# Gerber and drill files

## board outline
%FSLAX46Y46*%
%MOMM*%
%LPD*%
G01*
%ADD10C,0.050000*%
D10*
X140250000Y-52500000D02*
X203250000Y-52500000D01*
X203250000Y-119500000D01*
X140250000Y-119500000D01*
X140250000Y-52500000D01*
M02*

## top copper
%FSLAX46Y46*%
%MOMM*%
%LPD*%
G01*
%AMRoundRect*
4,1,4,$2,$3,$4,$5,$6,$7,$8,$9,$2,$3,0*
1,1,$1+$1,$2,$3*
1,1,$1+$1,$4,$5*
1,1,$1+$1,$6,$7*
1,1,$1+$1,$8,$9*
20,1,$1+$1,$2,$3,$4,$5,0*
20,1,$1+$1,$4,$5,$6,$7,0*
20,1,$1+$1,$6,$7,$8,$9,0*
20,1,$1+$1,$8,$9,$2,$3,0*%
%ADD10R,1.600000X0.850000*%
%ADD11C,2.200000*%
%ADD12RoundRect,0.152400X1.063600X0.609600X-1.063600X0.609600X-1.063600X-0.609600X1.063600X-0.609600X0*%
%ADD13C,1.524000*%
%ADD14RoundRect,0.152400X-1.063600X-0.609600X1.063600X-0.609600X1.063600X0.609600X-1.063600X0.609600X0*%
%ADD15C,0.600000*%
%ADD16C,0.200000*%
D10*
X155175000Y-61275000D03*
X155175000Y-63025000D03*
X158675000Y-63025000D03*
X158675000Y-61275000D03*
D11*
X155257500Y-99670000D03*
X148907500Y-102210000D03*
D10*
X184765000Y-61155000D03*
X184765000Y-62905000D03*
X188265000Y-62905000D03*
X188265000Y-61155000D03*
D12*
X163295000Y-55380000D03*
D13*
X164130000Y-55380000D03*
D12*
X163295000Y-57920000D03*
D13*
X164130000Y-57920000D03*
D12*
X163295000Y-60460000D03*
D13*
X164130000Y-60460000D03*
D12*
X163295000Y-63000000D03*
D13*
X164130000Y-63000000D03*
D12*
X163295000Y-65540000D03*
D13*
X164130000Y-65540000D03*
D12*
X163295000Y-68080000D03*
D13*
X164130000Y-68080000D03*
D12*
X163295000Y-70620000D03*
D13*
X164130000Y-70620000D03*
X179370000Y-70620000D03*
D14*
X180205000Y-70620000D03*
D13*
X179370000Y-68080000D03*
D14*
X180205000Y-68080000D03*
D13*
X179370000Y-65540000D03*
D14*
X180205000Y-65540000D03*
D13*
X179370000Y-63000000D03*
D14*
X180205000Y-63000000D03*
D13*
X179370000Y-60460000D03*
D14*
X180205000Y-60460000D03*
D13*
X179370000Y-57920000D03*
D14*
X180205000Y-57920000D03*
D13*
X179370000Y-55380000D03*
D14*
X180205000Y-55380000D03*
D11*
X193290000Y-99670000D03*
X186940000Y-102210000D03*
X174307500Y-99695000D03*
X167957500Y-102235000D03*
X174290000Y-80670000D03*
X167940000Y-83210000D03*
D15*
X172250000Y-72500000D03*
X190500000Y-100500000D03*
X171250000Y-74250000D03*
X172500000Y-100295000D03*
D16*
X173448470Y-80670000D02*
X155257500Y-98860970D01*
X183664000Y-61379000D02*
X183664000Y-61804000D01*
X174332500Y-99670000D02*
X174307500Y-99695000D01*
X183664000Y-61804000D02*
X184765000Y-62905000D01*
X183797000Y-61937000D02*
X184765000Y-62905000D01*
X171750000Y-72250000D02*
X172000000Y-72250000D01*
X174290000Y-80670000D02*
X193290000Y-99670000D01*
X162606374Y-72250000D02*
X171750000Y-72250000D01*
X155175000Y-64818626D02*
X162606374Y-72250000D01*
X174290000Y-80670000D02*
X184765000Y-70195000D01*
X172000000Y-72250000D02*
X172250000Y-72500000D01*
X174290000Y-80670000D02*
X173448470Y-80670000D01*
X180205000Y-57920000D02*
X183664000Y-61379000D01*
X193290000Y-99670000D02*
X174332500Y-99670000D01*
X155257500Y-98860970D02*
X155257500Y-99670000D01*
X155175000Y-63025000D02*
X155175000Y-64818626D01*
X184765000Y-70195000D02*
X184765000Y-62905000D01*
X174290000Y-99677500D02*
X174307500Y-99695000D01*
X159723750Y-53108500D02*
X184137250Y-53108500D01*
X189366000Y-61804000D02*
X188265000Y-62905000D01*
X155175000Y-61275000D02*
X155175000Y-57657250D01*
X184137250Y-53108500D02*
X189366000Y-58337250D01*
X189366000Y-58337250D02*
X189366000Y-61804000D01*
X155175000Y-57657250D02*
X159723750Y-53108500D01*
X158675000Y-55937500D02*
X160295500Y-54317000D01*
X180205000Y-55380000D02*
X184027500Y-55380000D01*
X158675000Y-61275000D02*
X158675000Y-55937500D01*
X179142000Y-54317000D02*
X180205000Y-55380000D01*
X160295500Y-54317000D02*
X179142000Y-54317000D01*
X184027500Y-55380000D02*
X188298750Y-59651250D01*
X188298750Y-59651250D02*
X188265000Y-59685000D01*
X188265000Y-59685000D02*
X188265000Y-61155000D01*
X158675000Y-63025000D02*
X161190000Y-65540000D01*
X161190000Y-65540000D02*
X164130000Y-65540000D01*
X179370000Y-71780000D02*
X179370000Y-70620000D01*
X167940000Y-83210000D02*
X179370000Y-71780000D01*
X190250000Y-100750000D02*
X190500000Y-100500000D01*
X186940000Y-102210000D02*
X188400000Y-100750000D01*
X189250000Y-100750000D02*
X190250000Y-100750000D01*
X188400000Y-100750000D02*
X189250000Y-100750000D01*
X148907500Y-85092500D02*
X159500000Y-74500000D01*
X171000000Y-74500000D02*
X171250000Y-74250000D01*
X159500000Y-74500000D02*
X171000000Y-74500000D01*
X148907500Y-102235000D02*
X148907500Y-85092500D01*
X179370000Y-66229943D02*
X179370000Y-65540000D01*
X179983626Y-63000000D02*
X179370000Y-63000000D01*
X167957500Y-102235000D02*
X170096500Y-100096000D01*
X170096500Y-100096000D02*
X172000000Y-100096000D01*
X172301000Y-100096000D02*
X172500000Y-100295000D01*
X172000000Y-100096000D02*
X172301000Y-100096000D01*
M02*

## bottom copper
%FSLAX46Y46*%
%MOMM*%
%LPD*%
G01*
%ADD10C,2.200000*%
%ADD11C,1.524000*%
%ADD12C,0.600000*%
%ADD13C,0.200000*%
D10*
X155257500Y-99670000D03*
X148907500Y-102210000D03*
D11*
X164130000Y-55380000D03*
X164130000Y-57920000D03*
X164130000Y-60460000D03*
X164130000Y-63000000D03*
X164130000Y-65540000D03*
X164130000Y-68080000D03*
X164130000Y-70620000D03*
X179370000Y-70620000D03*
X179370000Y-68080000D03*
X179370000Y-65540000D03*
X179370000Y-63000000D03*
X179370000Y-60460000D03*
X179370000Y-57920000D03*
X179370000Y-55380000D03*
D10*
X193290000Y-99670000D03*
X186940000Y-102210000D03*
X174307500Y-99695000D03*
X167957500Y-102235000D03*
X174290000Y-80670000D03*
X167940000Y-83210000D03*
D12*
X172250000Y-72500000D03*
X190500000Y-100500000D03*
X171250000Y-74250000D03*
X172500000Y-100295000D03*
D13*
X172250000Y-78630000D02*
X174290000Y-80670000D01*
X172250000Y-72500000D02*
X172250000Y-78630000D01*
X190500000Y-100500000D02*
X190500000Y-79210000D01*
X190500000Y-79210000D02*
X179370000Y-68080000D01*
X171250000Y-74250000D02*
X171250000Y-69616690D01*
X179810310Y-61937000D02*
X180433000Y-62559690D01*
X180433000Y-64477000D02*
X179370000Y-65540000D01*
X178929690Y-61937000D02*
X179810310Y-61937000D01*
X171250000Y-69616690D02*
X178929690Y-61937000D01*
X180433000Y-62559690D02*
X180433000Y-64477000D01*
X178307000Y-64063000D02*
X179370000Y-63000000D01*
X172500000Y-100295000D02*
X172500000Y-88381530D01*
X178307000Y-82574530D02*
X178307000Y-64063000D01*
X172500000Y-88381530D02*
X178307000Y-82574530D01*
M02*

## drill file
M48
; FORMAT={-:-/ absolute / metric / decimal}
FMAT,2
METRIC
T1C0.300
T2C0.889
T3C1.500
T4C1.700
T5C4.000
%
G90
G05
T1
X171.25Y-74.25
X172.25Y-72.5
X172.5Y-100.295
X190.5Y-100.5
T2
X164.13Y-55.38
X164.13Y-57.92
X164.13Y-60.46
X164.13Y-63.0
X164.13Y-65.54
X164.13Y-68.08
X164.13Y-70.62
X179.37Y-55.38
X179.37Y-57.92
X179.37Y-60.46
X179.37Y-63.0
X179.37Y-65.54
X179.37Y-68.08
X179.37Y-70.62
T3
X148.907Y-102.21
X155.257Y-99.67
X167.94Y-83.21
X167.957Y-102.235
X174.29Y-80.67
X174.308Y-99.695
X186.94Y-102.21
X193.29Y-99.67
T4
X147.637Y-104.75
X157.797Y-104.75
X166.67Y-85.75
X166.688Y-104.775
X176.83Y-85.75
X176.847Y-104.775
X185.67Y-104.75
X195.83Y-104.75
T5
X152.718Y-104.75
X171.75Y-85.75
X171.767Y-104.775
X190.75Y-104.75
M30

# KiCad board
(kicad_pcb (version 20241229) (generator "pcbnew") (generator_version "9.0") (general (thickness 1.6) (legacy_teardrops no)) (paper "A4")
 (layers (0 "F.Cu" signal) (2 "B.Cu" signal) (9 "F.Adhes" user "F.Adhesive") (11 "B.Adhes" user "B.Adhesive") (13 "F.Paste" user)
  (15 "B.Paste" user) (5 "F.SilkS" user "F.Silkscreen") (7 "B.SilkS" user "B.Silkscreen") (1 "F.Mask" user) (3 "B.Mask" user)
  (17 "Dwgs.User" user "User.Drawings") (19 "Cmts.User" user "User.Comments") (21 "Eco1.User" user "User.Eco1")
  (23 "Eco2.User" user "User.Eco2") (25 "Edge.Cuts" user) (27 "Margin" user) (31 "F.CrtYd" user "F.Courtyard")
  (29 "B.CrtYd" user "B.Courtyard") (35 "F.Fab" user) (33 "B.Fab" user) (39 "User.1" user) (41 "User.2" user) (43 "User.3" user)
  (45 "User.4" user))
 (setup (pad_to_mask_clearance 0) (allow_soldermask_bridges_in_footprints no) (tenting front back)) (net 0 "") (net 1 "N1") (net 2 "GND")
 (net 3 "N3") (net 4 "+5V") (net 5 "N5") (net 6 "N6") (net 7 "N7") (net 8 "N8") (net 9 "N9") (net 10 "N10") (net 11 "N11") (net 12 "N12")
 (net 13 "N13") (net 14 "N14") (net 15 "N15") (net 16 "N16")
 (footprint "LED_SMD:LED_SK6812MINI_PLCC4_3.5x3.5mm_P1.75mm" (layer "F.Cu") (at 156.925 62.15)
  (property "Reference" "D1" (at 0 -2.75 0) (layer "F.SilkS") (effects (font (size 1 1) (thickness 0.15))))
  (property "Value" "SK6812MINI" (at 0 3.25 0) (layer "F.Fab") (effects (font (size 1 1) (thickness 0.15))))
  (pad "1" smd rect (at -1.75 -0.875) (size 1.6 0.85) (layers "F.Cu" "F.Mask" "F.Paste") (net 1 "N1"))
  (pad "2" smd rect (at -1.75 0.875) (size 1.6 0.85) (layers "F.Cu" "F.Mask" "F.Paste") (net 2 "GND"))
  (pad "3" smd rect (at 1.75 0.875) (size 1.6 0.85) (layers "F.Cu" "F.Mask" "F.Paste") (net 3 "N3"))
  (pad "4" smd rect (at 1.75 -0.875) (size 1.6 0.85) (layers "F.Cu" "F.Mask" "F.Paste") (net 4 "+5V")))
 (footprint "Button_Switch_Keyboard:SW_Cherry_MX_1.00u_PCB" (layer "F.Cu") (at 155.2575 99.67)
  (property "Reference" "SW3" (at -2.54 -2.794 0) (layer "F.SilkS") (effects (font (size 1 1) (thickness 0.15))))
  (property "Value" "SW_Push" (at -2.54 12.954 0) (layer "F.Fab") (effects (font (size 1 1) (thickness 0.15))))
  (pad "" np_thru_hole circle (at -7.62 5.08) (size 1.7 1.7) (drill 1.7) (layers "*.Cu" "*.Mask"))
  (pad "" np_thru_hole circle (at -2.54 5.08) (size 4 4) (drill 4) (layers "*.Cu" "*.Mask"))
  (pad "" np_thru_hole circle (at 2.54 5.08) (size 1.7 1.7) (drill 1.7) (layers "*.Cu" "*.Mask"))
  (pad "1" thru_hole circle (at 0 0) (size 2.2 2.2) (drill 1.5) (layers "*.Cu" "*.Mask") (remove_unused_layers no) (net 2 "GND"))
  (pad "2" thru_hole circle (at -6.35 2.54) (size 2.2 2.2) (drill 1.5) (layers "*.Cu" "*.Mask") (remove_unused_layers no) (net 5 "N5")))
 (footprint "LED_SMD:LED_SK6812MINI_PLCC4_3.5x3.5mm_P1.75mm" (layer "F.Cu") (at 186.515 62.03)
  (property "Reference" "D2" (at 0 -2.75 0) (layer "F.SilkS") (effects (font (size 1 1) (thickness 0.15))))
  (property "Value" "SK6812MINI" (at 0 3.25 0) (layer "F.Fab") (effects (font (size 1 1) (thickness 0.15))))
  (pad "1" smd rect (at -1.75 -0.875) (size 1.6 0.85) (layers "F.Cu" "F.Mask" "F.Paste") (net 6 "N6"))
  (pad "2" smd rect (at -1.75 0.875) (size 1.6 0.85) (layers "F.Cu" "F.Mask" "F.Paste") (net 2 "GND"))
  (pad "3" smd rect (at 1.75 0.875) (size 1.6 0.85) (layers "F.Cu" "F.Mask" "F.Paste") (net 1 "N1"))
  (pad "4" smd rect (at 1.75 -0.875) (size 1.6 0.85) (layers "F.Cu" "F.Mask" "F.Paste") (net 4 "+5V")))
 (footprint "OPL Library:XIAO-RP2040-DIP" (layer "F.Cu") (at 171.75 63)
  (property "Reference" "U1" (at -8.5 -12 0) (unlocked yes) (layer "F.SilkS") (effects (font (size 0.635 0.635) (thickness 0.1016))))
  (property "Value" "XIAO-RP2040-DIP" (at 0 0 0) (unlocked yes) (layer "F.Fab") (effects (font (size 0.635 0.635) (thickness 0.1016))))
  (pad "1" smd roundrect (at -8.455 -7.62 180) (size 2.432 1.524) (layers "F.Cu" "F.Mask") (roundrect_rratio 0.1) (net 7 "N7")
   (thermal_bridge_angle 45))
  (pad "1" thru_hole circle (at -7.62 -7.62 180) (size 1.524 1.524) (drill 0.889) (layers "*.Cu" "*.Mask") (remove_unused_layers no)
   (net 7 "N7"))
  (pad "2" smd roundrect (at -8.455 -5.08 180) (size 2.432 1.524) (layers "F.Cu" "F.Mask") (roundrect_rratio 0.1) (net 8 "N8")
   (thermal_bridge_angle 45))
  (pad "2" thru_hole circle (at -7.62 -5.08 180) (size 1.524 1.524) (drill 0.889) (layers "*.Cu" "*.Mask") (remove_unused_layers no)
   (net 8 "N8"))
  (pad "3" smd roundrect (at -8.455 -2.54 180) (size 2.432 1.524) (layers "F.Cu" "F.Mask") (roundrect_rratio 0.1) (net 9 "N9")
   (thermal_bridge_angle 45))
  (pad "3" thru_hole circle (at -7.62 -2.54 180) (size 1.524 1.524) (drill 0.889) (layers "*.Cu" "*.Mask") (remove_unused_layers no)
   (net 9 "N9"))
  (pad "4" smd roundrect (at -8.455 0 180) (size 2.432 1.524) (layers "F.Cu" "F.Mask") (roundrect_rratio 0.1) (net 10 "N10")
   (thermal_bridge_angle 45))
  (pad "4" thru_hole circle (at -7.62 0 180) (size 1.524 1.524) (drill 0.889) (layers "*.Cu" "*.Mask") (remove_unused_layers no)
   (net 10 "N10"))
  (pad "5" smd roundrect (at -8.455 2.54 180) (size 2.432 1.524) (layers "F.Cu" "F.Mask") (roundrect_rratio 0.1) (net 3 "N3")
   (thermal_bridge_angle 45))
  (pad "5" thru_hole circle (at -7.62 2.54 180) (size 1.524 1.524) (drill 0.889) (layers "*.Cu" "*.Mask") (remove_unused_layers no)
   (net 3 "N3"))
  (pad "6" smd roundrect (at -8.455 5.08 180) (size 2.432 1.524) (layers "F.Cu" "F.Mask") (roundrect_rratio 0.1) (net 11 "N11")
   (thermal_bridge_angle 45))
  (pad "6" thru_hole circle (at -7.62 5.08 180) (size 1.524 1.524) (drill 0.889) (layers "*.Cu" "*.Mask") (remove_unused_layers no)
   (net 11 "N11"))
  (pad "7" smd roundrect (at -8.455 7.62 180) (size 2.432 1.524) (layers "F.Cu" "F.Mask") (roundrect_rratio 0.1) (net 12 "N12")
   (thermal_bridge_angle 45))
  (pad "7" thru_hole circle (at -7.62 7.62 180) (size 1.524 1.524) (drill 0.889) (layers "*.Cu" "*.Mask") (remove_unused_layers no)
   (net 12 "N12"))
  (pad "8" thru_hole circle (at 7.62 7.62) (size 1.524 1.524) (drill 0.889) (layers "*.Cu" "*.Mask") (remove_unused_layers no)
   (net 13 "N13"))
  (pad "8" smd roundrect (at 8.455 7.62) (size 2.432 1.524) (layers "F.Cu" "F.Mask") (roundrect_rratio 0.1) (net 13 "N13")
   (thermal_bridge_angle 45))
  (pad "9" thru_hole circle (at 7.62 5.08) (size 1.524 1.524) (drill 0.889) (layers "*.Cu" "*.Mask") (remove_unused_layers no)
   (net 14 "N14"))
  (pad "9" smd roundrect (at 8.455 5.08) (size 2.432 1.524) (layers "F.Cu" "F.Mask") (roundrect_rratio 0.1) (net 14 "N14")
   (thermal_bridge_angle 45))
  (pad "10" thru_hole circle (at 7.62 2.54) (size 1.524 1.524) (drill 0.889) (layers "*.Cu" "*.Mask") (remove_unused_layers no) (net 5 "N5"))
  (pad "10" smd roundrect (at 8.455 2.54) (size 2.432 1.524) (layers "F.Cu" "F.Mask") (roundrect_rratio 0.1) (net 5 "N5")
   (thermal_bridge_angle 45))
  (pad "11" thru_hole circle (at 7.62 0) (size 1.524 1.524) (drill 0.889) (layers "*.Cu" "*.Mask") (remove_unused_layers no) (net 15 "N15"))
  (pad "11" smd roundrect (at 8.455 0) (size 2.432 1.524) (layers "F.Cu" "F.Mask") (roundrect_rratio 0.1) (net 15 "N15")
   (thermal_bridge_angle 45))
  (pad "12" thru_hole circle (at 7.62 -2.54) (size 1.524 1.524) (drill 0.889) (layers "*.Cu" "*.Mask") (remove_unused_layers no)
   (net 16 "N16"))
  (pad "12" smd roundrect (at 8.455 -2.54) (size 2.432 1.524) (layers "F.Cu" "F.Mask") (roundrect_rratio 0.1) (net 16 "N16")
   (thermal_bridge_angle 45))
  (pad "13" thru_hole circle (at 7.62 -5.08) (size 1.524 1.524) (drill 0.889) (layers "*.Cu" "*.Mask") (remove_unused_layers no)
   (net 2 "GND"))
  (pad "13" smd roundrect (at 8.455 -5.08) (size 2.432 1.524) (layers "F.Cu" "F.Mask") (roundrect_rratio 0.1) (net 2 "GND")
   (thermal_bridge_angle 45))
  (pad "14" thru_hole circle (at 7.62 -7.62) (size 1.524 1.524) (drill 0.889) (layers "*.Cu" "*.Mask") (remove_unused_layers no)
   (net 4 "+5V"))
  (pad "14" smd roundrect (at 8.455 -7.62) (size 2.432 1.524) (layers "F.Cu" "F.Mask") (roundrect_rratio 0.1) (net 4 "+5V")
   (thermal_bridge_angle 45)))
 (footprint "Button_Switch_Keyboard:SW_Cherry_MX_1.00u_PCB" (layer "F.Cu") (at 193.29 99.67)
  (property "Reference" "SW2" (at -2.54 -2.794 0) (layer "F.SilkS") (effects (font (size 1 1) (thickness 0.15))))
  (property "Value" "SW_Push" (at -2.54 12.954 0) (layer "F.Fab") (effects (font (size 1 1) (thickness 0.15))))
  (pad "" np_thru_hole circle (at -7.62 5.08) (size 1.7 1.7) (drill 1.7) (layers "*.Cu" "*.Mask"))
  (pad "" np_thru_hole circle (at -2.54 5.08) (size 4 4) (drill 4) (layers "*.Cu" "*.Mask"))
  (pad "" np_thru_hole circle (at 2.54 5.08) (size 1.7 1.7) (drill 1.7) (layers "*.Cu" "*.Mask"))
  (pad "1" thru_hole circle (at 0 0) (size 2.2 2.2) (drill 1.5) (layers "*.Cu" "*.Mask") (remove_unused_layers no) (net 2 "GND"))
  (pad "2" thru_hole circle (at -6.35 2.54) (size 2.2 2.2) (drill 1.5) (layers "*.Cu" "*.Mask") (remove_unused_layers no) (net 14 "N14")))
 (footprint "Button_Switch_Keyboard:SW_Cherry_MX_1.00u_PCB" (layer "F.Cu") (at 174.3075 99.695)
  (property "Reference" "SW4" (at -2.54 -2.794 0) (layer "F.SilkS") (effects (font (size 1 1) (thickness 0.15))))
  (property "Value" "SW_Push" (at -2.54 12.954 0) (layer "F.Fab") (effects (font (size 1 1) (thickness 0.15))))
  (pad "" np_thru_hole circle (at -7.62 5.08) (size 1.7 1.7) (drill 1.7) (layers "*.Cu" "*.Mask"))
  (pad "" np_thru_hole circle (at -2.54 5.08) (size 4 4) (drill 4) (layers "*.Cu" "*.Mask"))
  (pad "" np_thru_hole circle (at 2.54 5.08) (size 1.7 1.7) (drill 1.7) (layers "*.Cu" "*.Mask"))
  (pad "1" thru_hole circle (at 0 0) (size 2.2 2.2) (drill 1.5) (layers "*.Cu" "*.Mask") (remove_unused_layers no) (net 2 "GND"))
  (pad "2" thru_hole circle (at -6.35 2.54) (size 2.2 2.2) (drill 1.5) (layers "*.Cu" "*.Mask") (remove_unused_layers no) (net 15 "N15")))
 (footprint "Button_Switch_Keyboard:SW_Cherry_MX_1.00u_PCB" (layer "F.Cu") (at 174.29 80.67)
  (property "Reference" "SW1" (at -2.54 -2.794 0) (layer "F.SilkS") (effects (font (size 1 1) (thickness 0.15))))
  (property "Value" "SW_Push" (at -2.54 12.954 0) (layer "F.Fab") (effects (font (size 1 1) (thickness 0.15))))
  (pad "" np_thru_hole circle (at -7.62 5.08) (size 1.7 1.7) (drill 1.7) (layers "*.Cu" "*.Mask"))
  (pad "" np_thru_hole circle (at -2.54 5.08) (size 4 4) (drill 4) (layers "*.Cu" "*.Mask"))
  (pad "" np_thru_hole circle (at 2.54 5.08) (size 1.7 1.7) (drill 1.7) (layers "*.Cu" "*.Mask"))
  (pad "1" thru_hole circle (at 0 0) (size 2.2 2.2) (drill 1.5) (layers "*.Cu" "*.Mask") (remove_unused_layers no) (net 2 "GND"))
  (pad "2" thru_hole circle (at -6.35 2.54) (size 2.2 2.2) (drill 1.5) (layers "*.Cu" "*.Mask") (remove_unused_layers no) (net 13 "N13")))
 (gr_rect (start 140.25 52.5) (end 203.25 119.5) (stroke (width 0.05) (type solid)) (fill no) (layer "Edge.Cuts"))
 (segment (start 173.44847 80.67) (end 155.2575 98.86097) (width 0.2) (layer "F.Cu") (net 2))
 (segment (start 183.664 61.379) (end 183.664 61.804) (width 0.2) (layer "F.Cu") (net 2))
 (segment (start 174.3325 99.67) (end 174.3075 99.695) (width 0.2) (layer "F.Cu") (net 2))
 (segment (start 183.664 61.804) (end 184.765 62.905) (width 0.2) (layer "F.Cu") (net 2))
 (segment (start 183.797 61.937) (end 184.765 62.905) (width 0.2) (layer "F.Cu") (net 2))
 (segment (start 171.75 72.25) (end 172 72.25) (width 0.2) (layer "F.Cu") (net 2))
 (segment (start 174.29 80.67) (end 193.29 99.67) (width 0.2) (layer "F.Cu") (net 2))
 (segment (start 162.606374 72.25) (end 171.75 72.25) (width 0.2) (layer "F.Cu") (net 2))
 (segment (start 155.175 64.818626) (end 162.606374 72.25) (width 0.2) (layer "F.Cu") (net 2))
 (segment (start 174.29 80.67) (end 184.765 70.195) (width 0.2) (layer "F.Cu") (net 2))
 (segment (start 172 72.25) (end 172.25 72.5) (width 0.2) (layer "F.Cu") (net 2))
 (segment (start 174.29 80.67) (end 173.44847 80.67) (width 0.2) (layer "F.Cu") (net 2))
 (segment (start 180.205 57.92) (end 183.664 61.379) (width 0.2) (layer "F.Cu") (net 2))
 (segment (start 193.29 99.67) (end 174.3325 99.67) (width 0.2) (layer "F.Cu") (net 2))
 (segment (start 155.2575 98.86097) (end 155.2575 99.67) (width 0.2) (layer "F.Cu") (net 2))
 (segment (start 155.175 63.025) (end 155.175 64.818626) (width 0.2) (layer "F.Cu") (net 2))
 (segment (start 184.765 70.195) (end 184.765 62.905) (width 0.2) (layer "F.Cu") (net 2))
 (segment (start 174.29 99.6775) (end 174.3075 99.695) (width 0.2) (layer "F.Cu") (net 2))
 (via (at 172.25 72.5) (size 0.6) (drill 0.3) (layers "F.Cu" "B.Cu") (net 2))
 (segment (start 172.25 78.63) (end 174.29 80.67) (width 0.2) (layer "B.Cu") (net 2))
 (segment (start 172.25 72.5) (end 172.25 78.63) (width 0.2) (layer "B.Cu") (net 2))
 (segment (start 159.72375 53.1085) (end 184.13725 53.1085) (width 0.2) (layer "F.Cu") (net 1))
 (segment (start 189.366 61.804) (end 188.265 62.905) (width 0.2) (layer "F.Cu") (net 1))
 (segment (start 155.175 61.275) (end 155.175 57.65725) (width 0.2) (layer "F.Cu") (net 1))
 (segment (start 184.13725 53.1085) (end 189.366 58.33725) (width 0.2) (layer "F.Cu") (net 1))
 (segment (start 189.366 58.33725) (end 189.366 61.804) (width 0.2) (layer "F.Cu") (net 1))
 (segment (start 155.175 57.65725) (end 159.72375 53.1085) (width 0.2) (layer "F.Cu") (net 1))
 (segment (start 158.675 55.9375) (end 160.2955 54.317) (width 0.2) (layer "F.Cu") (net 4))
 (segment (start 180.205 55.38) (end 184.0275 55.38) (width 0.2) (layer "F.Cu") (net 4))
 (segment (start 158.675 61.275) (end 158.675 55.9375) (width 0.2) (layer "F.Cu") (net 4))
 (segment (start 179.142 54.317) (end 180.205 55.38) (width 0.2) (layer "F.Cu") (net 4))
 (segment (start 160.2955 54.317) (end 179.142 54.317) (width 0.2) (layer "F.Cu") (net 4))
 (segment (start 184.0275 55.38) (end 188.29875 59.65125) (width 0.2) (layer "F.Cu") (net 4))
 (segment (start 188.29875 59.65125) (end 188.265 59.685) (width 0.2) (layer "F.Cu") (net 4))
 (segment (start 188.265 59.685) (end 188.265 61.155) (width 0.2) (layer "F.Cu") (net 4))
 (segment (start 158.675 63.025) (end 161.19 65.54) (width 0.2) (layer "F.Cu") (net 3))
 (segment (start 161.19 65.54) (end 164.13 65.54) (width 0.2) (layer "F.Cu") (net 3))
 (segment (start 179.37 71.78) (end 179.37 70.62) (width 0.2) (layer "F.Cu") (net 13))
 (segment (start 167.94 83.21) (end 179.37 71.78) (width 0.2) (layer "F.Cu") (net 13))
 (segment (start 190.25 100.75) (end 190.5 100.5) (width 0.2) (layer "F.Cu") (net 14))
 (segment (start 186.94 102.21) (end 188.4 100.75) (width 0.2) (layer "F.Cu") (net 14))
 (segment (start 189.25 100.75) (end 190.25 100.75) (width 0.2) (layer "F.Cu") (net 14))
 (segment (start 188.4 100.75) (end 189.25 100.75) (width 0.2) (layer "F.Cu") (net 14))
 (via (at 190.5 100.5) (size 0.6) (drill 0.3) (layers "F.Cu" "B.Cu") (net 14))
 (segment (start 190.5 100.5) (end 190.5 79.21) (width 0.2) (layer "B.Cu") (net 14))
 (segment (start 190.5 79.21) (end 179.37 68.08) (width 0.2) (layer "B.Cu") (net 14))
 (segment (start 148.9075 85.0925) (end 159.5 74.5) (width 0.2) (layer "F.Cu") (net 5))
 (segment (start 171 74.5) (end 171.25 74.25) (width 0.2) (layer "F.Cu") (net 5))
 (segment (start 159.5 74.5) (end 171 74.5) (width 0.2) (layer "F.Cu") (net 5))
 (segment (start 148.9075 102.235) (end 148.9075 85.0925) (width 0.2) (layer "F.Cu") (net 5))
 (segment (start 179.37 66.229943) (end 179.37 65.54) (width 0.2) (layer "F.Cu") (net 5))
 (via (at 171.25 74.25) (size 0.6) (drill 0.3) (layers "F.Cu" "B.Cu") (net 5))
 (segment (start 171.25 74.25) (end 171.25 69.61669) (width 0.2) (layer "B.Cu") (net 5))
 (segment (start 179.81031 61.937) (end 180.433 62.55969) (width 0.2) (layer "B.Cu") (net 5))
 (segment (start 180.433 64.477) (end 179.37 65.54) (width 0.2) (layer "B.Cu") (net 5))
 (segment (start 178.92969 61.937) (end 179.81031 61.937) (width 0.2) (layer "B.Cu") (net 5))
 (segment (start 171.25 69.61669) (end 178.92969 61.937) (width 0.2) (layer "B.Cu") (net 5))
 (segment (start 180.433 62.55969) (end 180.433 64.477) (width 0.2) (layer "B.Cu") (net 5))
 (segment (start 179.983626 63) (end 179.37 63) (width 0.2) (layer "F.Cu") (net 15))
 (segment (start 167.9575 102.235) (end 170.0965 100.096) (width 0.2) (layer "F.Cu") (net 15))
 (segment (start 170.0965 100.096) (end 172 100.096) (width 0.2) (layer "F.Cu") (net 15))
 (segment (start 172.301 100.096) (end 172.5 100.295) (width 0.2) (layer "F.Cu") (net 15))
 (segment (start 172 100.096) (end 172.301 100.096) (width 0.2) (layer "F.Cu") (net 15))
 (via (at 172.5 100.295) (size 0.6) (drill 0.3) (layers "F.Cu" "B.Cu") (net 15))
 (segment (start 178.307 64.063) (end 179.37 63) (width 0.2) (layer "B.Cu") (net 15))
 (segment (start 172.5 100.295) (end 172.5 88.38153) (width 0.2) (layer "B.Cu") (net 15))
 (segment (start 178.307 82.57453) (end 178.307 64.063) (width 0.2) (layer "B.Cu") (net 15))
 (segment (start 172.5 88.38153) (end 178.307 82.57453) (width 0.2) (layer "B.Cu") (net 15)))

